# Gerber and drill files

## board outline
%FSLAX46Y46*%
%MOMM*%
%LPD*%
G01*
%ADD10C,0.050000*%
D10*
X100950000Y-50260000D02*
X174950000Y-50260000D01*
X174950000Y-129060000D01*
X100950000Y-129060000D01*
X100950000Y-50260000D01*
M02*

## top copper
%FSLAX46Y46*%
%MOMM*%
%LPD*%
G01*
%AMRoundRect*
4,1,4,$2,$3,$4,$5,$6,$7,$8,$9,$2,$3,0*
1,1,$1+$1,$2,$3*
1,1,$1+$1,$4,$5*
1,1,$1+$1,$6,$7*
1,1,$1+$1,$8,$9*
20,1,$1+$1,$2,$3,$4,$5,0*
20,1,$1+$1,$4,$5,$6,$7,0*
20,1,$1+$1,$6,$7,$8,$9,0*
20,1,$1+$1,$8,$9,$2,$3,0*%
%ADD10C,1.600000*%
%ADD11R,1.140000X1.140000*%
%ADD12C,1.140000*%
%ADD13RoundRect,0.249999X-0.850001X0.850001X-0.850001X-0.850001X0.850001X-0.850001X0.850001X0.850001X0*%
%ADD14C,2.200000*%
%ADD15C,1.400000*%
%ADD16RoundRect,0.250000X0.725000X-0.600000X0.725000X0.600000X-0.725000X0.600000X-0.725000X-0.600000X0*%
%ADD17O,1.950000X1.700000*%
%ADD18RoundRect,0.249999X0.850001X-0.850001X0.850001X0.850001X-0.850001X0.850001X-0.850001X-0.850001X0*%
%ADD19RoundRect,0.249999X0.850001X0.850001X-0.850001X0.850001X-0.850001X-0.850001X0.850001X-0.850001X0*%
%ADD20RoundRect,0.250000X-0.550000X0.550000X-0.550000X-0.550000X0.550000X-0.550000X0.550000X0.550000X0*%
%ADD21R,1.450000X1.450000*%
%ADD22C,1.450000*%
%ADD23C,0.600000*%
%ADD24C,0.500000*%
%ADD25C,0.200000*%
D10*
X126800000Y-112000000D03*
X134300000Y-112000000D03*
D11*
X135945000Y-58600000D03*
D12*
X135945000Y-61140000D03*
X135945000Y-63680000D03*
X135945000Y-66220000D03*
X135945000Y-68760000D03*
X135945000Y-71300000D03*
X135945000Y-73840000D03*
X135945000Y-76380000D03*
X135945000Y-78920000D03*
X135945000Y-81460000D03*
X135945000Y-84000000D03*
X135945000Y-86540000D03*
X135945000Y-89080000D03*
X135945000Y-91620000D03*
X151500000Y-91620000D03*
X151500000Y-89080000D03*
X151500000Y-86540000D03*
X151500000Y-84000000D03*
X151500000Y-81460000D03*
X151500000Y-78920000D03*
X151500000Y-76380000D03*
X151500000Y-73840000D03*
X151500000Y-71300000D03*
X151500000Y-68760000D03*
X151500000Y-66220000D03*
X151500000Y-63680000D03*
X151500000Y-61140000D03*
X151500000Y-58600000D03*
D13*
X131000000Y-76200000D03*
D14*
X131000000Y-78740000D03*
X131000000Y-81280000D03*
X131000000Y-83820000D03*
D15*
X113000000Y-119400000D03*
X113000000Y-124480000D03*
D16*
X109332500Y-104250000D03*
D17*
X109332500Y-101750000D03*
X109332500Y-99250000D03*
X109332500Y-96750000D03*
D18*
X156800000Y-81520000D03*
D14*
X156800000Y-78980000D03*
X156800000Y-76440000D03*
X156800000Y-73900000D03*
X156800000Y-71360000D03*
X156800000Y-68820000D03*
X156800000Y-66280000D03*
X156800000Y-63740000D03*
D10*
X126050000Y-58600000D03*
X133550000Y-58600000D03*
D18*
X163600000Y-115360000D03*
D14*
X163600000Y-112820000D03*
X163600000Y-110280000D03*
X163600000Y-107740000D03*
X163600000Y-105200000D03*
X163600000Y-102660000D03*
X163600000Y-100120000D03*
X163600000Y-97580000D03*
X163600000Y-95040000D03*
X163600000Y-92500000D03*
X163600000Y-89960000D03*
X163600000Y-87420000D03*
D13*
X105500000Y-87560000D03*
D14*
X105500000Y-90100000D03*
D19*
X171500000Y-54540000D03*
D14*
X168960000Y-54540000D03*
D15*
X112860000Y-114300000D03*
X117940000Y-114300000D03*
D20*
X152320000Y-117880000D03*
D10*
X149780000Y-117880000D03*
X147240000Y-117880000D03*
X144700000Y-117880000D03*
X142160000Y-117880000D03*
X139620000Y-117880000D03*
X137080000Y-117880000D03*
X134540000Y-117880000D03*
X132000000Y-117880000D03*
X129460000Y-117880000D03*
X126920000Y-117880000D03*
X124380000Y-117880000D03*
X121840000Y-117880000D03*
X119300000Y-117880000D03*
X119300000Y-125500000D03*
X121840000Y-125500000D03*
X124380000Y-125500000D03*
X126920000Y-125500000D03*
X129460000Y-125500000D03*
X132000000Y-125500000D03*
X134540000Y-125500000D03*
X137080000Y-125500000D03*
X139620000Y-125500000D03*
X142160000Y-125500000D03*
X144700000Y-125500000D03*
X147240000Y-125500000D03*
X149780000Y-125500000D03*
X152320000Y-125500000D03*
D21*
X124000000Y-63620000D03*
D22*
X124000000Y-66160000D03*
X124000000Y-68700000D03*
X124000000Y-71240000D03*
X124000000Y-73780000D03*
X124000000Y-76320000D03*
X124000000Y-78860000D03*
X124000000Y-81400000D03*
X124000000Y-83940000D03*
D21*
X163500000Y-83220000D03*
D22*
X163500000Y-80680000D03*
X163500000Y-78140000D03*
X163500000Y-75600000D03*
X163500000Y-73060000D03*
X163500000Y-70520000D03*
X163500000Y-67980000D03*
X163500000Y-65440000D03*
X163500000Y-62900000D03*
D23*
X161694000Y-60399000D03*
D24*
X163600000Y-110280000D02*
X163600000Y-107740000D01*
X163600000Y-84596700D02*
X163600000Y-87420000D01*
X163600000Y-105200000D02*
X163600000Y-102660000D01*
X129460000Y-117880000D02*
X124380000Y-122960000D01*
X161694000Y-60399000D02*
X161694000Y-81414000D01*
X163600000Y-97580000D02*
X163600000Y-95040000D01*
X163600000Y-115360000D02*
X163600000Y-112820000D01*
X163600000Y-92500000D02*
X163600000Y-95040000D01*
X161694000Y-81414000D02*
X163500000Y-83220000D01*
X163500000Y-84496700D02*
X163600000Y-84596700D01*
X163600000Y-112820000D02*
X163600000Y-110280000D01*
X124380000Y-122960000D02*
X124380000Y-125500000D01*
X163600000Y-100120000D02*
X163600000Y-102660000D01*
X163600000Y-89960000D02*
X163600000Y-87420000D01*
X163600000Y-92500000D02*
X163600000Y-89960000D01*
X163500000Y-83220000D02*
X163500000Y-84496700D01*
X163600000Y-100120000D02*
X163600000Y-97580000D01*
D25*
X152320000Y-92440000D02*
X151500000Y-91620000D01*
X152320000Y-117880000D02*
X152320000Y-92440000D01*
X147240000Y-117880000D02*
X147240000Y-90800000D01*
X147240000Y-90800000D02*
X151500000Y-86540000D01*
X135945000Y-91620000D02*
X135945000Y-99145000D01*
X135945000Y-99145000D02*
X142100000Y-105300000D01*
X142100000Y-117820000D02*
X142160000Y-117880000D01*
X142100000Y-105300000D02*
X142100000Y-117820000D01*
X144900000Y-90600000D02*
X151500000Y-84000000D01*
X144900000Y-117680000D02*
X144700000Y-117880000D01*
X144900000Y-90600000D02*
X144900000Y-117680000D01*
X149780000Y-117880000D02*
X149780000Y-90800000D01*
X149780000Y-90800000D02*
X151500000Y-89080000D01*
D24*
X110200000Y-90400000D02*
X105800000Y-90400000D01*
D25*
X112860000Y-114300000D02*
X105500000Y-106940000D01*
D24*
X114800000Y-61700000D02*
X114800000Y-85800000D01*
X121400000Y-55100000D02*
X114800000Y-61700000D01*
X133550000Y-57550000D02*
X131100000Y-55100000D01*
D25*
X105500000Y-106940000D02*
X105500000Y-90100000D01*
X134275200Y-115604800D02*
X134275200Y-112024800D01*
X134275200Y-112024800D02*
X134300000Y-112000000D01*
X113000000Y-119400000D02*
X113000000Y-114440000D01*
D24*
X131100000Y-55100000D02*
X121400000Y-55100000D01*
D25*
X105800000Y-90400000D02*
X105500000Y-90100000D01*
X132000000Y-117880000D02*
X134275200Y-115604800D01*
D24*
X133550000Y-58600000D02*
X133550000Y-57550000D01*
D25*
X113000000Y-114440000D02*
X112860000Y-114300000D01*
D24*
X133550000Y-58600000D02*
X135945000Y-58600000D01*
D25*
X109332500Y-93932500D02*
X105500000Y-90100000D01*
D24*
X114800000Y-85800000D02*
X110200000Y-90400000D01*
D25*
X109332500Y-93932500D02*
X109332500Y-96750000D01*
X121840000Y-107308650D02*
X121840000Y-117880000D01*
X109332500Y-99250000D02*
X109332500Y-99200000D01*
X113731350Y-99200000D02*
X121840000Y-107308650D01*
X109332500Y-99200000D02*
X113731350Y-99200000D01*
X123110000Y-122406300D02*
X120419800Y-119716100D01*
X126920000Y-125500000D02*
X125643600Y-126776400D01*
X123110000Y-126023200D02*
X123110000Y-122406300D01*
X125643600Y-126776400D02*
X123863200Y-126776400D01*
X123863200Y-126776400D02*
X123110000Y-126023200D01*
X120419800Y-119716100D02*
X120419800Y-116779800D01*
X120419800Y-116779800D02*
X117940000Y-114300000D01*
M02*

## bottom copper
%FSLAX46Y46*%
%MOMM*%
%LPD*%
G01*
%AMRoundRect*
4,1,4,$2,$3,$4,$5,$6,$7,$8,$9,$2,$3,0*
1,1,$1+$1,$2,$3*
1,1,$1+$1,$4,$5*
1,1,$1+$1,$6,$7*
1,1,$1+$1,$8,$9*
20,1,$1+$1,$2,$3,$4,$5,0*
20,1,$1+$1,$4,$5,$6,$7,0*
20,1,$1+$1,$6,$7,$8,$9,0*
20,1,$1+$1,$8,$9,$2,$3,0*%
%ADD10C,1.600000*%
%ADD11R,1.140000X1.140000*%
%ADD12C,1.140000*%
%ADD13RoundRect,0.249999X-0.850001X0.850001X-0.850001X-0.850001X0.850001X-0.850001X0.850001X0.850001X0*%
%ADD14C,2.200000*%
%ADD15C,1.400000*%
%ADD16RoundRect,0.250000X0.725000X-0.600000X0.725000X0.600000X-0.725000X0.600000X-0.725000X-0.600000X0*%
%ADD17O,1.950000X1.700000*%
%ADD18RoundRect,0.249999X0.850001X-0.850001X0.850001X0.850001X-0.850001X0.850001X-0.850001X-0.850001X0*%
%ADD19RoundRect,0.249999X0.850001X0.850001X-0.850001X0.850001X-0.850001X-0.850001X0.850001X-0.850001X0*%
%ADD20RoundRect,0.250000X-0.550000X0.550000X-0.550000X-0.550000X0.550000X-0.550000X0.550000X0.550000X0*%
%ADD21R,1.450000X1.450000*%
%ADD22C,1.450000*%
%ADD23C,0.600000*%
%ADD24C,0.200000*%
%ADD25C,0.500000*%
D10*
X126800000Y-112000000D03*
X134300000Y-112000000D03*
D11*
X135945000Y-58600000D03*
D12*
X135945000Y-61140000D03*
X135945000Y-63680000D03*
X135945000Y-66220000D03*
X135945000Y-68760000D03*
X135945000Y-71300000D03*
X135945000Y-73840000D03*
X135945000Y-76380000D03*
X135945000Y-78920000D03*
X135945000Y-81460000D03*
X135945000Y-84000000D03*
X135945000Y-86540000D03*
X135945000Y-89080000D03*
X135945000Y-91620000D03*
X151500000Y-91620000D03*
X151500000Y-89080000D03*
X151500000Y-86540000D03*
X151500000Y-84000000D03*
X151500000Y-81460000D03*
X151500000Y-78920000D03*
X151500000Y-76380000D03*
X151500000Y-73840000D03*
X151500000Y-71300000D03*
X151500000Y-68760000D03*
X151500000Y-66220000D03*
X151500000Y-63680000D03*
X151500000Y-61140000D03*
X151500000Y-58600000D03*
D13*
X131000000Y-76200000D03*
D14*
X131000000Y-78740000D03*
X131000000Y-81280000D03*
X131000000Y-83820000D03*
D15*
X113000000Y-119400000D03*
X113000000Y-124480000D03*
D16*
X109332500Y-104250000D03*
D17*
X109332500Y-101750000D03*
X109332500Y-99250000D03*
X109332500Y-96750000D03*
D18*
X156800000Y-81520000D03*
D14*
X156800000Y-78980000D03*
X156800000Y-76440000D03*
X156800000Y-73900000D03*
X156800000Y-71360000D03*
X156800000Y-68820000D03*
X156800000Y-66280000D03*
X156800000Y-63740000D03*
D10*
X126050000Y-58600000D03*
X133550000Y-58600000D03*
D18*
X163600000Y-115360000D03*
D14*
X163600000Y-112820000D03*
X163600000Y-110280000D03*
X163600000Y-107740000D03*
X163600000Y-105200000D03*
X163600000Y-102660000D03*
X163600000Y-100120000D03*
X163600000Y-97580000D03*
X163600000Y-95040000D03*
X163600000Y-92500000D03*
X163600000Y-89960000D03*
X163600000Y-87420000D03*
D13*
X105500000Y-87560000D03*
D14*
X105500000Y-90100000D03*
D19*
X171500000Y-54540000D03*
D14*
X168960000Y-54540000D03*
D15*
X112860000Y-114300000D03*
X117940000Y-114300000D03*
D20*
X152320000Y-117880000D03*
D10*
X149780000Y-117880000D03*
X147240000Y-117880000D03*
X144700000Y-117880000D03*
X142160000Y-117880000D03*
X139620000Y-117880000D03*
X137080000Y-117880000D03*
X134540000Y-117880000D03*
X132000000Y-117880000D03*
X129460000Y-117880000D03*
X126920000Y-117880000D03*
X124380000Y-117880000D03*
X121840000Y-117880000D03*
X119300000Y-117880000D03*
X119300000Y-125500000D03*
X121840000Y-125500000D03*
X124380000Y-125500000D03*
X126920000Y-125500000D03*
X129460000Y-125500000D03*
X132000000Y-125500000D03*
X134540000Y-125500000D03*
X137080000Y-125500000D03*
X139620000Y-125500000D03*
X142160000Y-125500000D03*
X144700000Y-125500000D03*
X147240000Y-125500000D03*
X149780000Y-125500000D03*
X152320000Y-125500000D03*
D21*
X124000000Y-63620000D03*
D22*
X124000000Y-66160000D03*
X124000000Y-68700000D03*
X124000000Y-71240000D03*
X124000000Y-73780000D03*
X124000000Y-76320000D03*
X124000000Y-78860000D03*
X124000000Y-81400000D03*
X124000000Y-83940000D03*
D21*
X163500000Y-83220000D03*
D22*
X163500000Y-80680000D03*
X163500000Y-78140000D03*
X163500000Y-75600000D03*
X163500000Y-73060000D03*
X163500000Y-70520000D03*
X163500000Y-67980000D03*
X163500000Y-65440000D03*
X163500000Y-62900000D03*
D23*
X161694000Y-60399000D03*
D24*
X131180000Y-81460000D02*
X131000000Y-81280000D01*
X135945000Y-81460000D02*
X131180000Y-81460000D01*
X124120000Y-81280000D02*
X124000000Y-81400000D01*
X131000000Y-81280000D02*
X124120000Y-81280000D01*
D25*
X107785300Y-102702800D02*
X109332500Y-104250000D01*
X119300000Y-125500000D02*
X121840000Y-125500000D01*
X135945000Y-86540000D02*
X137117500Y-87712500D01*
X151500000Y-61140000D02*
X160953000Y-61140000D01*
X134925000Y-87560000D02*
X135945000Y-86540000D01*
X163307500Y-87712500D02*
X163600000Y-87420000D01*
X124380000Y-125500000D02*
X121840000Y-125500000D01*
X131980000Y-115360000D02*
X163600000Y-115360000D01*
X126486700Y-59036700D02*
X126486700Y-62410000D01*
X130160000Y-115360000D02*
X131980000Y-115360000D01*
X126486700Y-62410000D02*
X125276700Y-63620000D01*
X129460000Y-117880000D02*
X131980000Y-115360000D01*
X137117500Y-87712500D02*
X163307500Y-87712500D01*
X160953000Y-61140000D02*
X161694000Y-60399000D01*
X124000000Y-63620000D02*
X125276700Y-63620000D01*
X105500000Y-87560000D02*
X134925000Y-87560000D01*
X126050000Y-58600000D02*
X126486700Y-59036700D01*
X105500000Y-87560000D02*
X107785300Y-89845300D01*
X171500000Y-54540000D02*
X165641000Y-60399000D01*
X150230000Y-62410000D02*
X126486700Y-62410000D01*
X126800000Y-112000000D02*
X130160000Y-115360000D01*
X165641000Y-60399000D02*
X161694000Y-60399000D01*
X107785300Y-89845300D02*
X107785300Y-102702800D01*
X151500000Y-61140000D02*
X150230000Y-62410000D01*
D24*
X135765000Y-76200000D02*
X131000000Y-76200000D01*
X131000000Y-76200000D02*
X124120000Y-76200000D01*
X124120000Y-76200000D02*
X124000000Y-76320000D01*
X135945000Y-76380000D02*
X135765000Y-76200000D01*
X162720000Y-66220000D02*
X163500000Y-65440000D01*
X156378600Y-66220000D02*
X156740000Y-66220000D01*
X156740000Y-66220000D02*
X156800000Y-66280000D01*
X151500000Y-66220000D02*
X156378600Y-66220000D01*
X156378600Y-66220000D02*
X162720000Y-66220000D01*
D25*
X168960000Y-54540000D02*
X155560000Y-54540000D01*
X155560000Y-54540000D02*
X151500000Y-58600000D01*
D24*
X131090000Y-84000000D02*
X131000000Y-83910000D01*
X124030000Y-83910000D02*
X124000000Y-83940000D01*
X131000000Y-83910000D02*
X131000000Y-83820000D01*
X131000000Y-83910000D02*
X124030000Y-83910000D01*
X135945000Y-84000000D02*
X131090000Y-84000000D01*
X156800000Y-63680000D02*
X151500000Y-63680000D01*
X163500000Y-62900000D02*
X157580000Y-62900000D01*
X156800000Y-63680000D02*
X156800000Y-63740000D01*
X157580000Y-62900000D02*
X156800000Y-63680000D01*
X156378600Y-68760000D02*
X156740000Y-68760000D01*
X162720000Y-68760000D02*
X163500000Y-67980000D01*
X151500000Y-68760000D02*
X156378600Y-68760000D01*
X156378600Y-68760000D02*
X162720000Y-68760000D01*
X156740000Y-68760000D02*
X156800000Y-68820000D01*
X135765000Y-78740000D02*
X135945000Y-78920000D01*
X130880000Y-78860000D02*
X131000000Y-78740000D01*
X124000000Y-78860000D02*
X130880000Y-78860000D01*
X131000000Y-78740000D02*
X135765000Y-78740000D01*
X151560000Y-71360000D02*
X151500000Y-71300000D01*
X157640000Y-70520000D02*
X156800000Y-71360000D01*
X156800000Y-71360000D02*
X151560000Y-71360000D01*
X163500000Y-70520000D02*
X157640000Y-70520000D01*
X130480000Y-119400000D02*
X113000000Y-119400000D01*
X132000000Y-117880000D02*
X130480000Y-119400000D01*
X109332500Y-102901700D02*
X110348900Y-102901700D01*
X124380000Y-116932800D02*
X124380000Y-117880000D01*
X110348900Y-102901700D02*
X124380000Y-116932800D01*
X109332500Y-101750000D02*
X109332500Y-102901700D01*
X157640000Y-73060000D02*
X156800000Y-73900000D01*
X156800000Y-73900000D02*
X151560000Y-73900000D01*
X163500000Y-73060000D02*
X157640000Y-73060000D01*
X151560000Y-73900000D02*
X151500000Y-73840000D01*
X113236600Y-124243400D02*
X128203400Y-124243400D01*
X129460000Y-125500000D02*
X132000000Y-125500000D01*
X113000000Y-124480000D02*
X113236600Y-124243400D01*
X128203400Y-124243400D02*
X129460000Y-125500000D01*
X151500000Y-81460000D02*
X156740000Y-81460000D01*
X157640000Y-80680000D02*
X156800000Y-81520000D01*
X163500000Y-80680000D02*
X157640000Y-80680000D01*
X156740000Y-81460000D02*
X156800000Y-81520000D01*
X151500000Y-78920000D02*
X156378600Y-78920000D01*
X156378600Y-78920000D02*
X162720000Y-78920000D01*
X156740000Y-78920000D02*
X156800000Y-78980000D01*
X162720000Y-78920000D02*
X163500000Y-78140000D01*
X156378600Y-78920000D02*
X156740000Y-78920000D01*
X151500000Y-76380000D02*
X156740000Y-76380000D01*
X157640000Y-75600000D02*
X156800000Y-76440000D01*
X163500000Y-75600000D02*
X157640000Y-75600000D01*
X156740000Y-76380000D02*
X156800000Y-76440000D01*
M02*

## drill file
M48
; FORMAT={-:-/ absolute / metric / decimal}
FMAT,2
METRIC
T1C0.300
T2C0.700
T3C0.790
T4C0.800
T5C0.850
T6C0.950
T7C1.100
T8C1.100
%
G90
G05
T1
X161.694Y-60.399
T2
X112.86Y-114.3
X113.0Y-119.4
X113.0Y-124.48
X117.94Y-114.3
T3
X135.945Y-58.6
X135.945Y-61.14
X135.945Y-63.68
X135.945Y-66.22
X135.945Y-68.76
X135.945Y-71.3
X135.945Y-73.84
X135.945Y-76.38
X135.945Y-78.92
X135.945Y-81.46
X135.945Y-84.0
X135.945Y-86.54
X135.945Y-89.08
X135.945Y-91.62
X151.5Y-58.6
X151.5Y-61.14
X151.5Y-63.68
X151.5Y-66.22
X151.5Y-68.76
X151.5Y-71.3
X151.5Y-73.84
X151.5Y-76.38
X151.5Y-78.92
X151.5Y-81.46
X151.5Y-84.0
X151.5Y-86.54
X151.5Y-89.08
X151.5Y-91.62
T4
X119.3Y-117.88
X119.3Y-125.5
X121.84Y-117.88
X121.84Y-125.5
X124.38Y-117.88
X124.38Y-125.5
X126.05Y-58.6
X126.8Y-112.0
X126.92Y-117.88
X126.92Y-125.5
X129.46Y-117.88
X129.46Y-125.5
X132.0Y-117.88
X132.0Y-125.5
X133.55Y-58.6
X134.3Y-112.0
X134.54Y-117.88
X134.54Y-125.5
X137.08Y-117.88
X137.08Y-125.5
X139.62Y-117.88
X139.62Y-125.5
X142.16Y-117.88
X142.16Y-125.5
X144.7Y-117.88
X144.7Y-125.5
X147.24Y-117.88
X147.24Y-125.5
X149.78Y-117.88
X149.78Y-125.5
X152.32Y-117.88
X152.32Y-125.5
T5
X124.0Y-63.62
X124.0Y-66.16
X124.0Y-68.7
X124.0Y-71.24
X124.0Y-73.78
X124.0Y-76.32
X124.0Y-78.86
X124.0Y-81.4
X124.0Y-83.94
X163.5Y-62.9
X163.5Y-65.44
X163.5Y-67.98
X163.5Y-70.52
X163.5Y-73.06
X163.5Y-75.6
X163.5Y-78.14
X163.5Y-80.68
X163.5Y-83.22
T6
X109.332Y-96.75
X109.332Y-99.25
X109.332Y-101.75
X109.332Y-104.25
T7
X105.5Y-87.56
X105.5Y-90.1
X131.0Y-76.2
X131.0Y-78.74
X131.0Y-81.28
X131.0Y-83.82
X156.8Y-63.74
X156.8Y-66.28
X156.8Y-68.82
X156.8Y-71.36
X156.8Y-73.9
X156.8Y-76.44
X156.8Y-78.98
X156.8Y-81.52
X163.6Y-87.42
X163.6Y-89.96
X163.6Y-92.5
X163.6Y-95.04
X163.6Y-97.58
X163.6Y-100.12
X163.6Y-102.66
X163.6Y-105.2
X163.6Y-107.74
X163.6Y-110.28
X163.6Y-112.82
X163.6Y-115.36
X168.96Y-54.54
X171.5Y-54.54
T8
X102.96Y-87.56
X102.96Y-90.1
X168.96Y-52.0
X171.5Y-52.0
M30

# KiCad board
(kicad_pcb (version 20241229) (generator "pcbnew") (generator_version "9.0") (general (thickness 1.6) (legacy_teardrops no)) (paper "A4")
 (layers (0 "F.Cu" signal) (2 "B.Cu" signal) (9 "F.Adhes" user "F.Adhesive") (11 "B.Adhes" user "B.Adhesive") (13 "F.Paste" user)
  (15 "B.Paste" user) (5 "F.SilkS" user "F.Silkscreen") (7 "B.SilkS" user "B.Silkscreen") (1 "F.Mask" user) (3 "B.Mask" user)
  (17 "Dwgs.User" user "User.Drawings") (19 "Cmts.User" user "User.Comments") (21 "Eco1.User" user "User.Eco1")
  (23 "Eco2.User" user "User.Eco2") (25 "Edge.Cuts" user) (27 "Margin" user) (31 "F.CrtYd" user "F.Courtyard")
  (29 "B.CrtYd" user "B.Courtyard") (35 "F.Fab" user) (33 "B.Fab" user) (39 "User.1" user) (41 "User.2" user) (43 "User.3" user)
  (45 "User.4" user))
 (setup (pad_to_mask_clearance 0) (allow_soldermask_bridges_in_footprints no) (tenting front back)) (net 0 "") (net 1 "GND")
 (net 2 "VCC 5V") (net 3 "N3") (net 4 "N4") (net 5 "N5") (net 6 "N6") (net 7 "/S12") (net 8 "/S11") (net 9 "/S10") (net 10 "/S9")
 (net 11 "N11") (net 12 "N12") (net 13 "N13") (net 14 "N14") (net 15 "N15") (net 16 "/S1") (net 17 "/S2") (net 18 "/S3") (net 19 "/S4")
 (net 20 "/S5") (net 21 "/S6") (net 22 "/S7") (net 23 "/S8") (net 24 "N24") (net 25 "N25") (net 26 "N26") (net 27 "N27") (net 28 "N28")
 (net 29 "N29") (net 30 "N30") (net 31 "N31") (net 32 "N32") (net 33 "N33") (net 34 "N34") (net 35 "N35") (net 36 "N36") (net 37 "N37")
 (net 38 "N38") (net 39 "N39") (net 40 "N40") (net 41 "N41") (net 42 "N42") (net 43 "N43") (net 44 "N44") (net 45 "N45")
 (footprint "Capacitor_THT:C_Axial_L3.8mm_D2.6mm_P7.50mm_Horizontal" (layer "F.Cu") (at 126.8 112)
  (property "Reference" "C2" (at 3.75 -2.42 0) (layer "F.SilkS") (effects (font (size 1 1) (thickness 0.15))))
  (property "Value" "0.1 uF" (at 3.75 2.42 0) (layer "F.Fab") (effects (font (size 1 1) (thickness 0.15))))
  (pad "1" thru_hole circle (at 0 0) (size 1.6 1.6) (drill 0.8) (layers "*.Cu" "*.Mask") (remove_unused_layers no) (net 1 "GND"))
  (pad "2" thru_hole circle (at 7.5 0) (size 1.6 1.6) (drill 0.8) (layers "*.Cu" "*.Mask") (remove_unused_layers no) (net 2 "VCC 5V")))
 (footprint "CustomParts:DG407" (layer "F.Cu") (at 143.7225 75.11)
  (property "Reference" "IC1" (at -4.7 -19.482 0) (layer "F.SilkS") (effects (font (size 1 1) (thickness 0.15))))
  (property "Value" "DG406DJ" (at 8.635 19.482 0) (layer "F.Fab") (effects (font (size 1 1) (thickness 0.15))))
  (pad "1" thru_hole rect (at -7.7775 -16.51) (size 1.14 1.14) (drill 0.79) (layers "*.Cu" "*.Mask") (remove_unused_layers no)
   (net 2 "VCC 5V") (solder_mask_margin 0.102))
  (pad "2" thru_hole circle (at -7.7775 -13.97) (size 1.14 1.14) (drill 0.79) (layers "*.Cu" "*.Mask") (remove_unused_layers no)
   (solder_mask_margin 0.102))
  (pad "3" thru_hole circle (at -7.7775 -11.43) (size 1.14 1.14) (drill 0.79) (layers "*.Cu" "*.Mask") (remove_unused_layers no)
   (solder_mask_margin 0.102))
  (pad "4" thru_hole circle (at -7.7775 -8.89) (size 1.14 1.14) (drill 0.79) (layers "*.Cu" "*.Mask") (remove_unused_layers no) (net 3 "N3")
   (solder_mask_margin 0.102))
  (pad "5" thru_hole circle (at -7.7775 -6.35) (size 1.14 1.14) (drill 0.79) (layers "*.Cu" "*.Mask") (remove_unused_layers no) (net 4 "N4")
   (solder_mask_margin 0.102))
  (pad "6" thru_hole circle (at -7.7775 -3.81) (size 1.14 1.14) (drill 0.79) (layers "*.Cu" "*.Mask") (remove_unused_layers no) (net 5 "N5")
   (solder_mask_margin 0.102))
  (pad "7" thru_hole circle (at -7.7775 -1.27) (size 1.14 1.14) (drill 0.79) (layers "*.Cu" "*.Mask") (remove_unused_layers no) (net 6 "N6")
   (solder_mask_margin 0.102))
  (pad "8" thru_hole circle (at -7.7775 1.27) (size 1.14 1.14) (drill 0.79) (layers "*.Cu" "*.Mask") (remove_unused_layers no)
   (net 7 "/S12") (solder_mask_margin 0.102))
  (pad "9" thru_hole circle (at -7.7775 3.81) (size 1.14 1.14) (drill 0.79) (layers "*.Cu" "*.Mask") (remove_unused_layers no)
   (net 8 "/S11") (solder_mask_margin 0.102))
  (pad "10" thru_hole circle (at -7.7775 6.35) (size 1.14 1.14) (drill 0.79) (layers "*.Cu" "*.Mask") (remove_unused_layers no)
   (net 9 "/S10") (solder_mask_margin 0.102))
  (pad "11" thru_hole circle (at -7.7775 8.89) (size 1.14 1.14) (drill 0.79) (layers "*.Cu" "*.Mask") (remove_unused_layers no)
   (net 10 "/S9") (solder_mask_margin 0.102))
  (pad "12" thru_hole circle (at -7.7775 11.43) (size 1.14 1.14) (drill 0.79) (layers "*.Cu" "*.Mask") (remove_unused_layers no)
   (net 1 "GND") (solder_mask_margin 0.102))
  (pad "13" thru_hole circle (at -7.7775 13.97) (size 1.14 1.14) (drill 0.79) (layers "*.Cu" "*.Mask") (remove_unused_layers no)
   (solder_mask_margin 0.102))
  (pad "14" thru_hole circle (at -7.7775 16.51) (size 1.14 1.14) (drill 0.79) (layers "*.Cu" "*.Mask") (remove_unused_layers no)
   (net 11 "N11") (solder_mask_margin 0.102))
  (pad "15" thru_hole circle (at 7.7775 16.51) (size 1.14 1.14) (drill 0.79) (layers "*.Cu" "*.Mask") (remove_unused_layers no)
   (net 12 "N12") (solder_mask_margin 0.102))
  (pad "16" thru_hole circle (at 7.7775 13.97) (size 1.14 1.14) (drill 0.79) (layers "*.Cu" "*.Mask") (remove_unused_layers no)
   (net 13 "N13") (solder_mask_margin 0.102))
  (pad "17" thru_hole circle (at 7.7775 11.43) (size 1.14 1.14) (drill 0.79) (layers "*.Cu" "*.Mask") (remove_unused_layers no)
   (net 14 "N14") (solder_mask_margin 0.102))
  (pad "18" thru_hole circle (at 7.7775 8.89) (size 1.14 1.14) (drill 0.79) (layers "*.Cu" "*.Mask") (remove_unused_layers no)
   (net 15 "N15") (solder_mask_margin 0.102))
  (pad "19" thru_hole circle (at 7.7775 6.35) (size 1.14 1.14) (drill 0.79) (layers "*.Cu" "*.Mask") (remove_unused_layers no)
   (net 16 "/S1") (solder_mask_margin 0.102))
  (pad "20" thru_hole circle (at 7.7775 3.81) (size 1.14 1.14) (drill 0.79) (layers "*.Cu" "*.Mask") (remove_unused_layers no)
   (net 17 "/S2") (solder_mask_margin 0.102))
  (pad "21" thru_hole circle (at 7.7775 1.27) (size 1.14 1.14) (drill 0.79) (layers "*.Cu" "*.Mask") (remove_unused_layers no)
   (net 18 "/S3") (solder_mask_margin 0.102))
  (pad "22" thru_hole circle (at 7.7775 -1.27) (size 1.14 1.14) (drill 0.79) (layers "*.Cu" "*.Mask") (remove_unused_layers no)
   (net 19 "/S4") (solder_mask_margin 0.102))
  (pad "23" thru_hole circle (at 7.7775 -3.81) (size 1.14 1.14) (drill 0.79) (layers "*.Cu" "*.Mask") (remove_unused_layers no)
   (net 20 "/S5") (solder_mask_margin 0.102))
  (pad "24" thru_hole circle (at 7.7775 -6.35) (size 1.14 1.14) (drill 0.79) (layers "*.Cu" "*.Mask") (remove_unused_layers no)
   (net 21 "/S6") (solder_mask_margin 0.102))
  (pad "25" thru_hole circle (at 7.7775 -8.89) (size 1.14 1.14) (drill 0.79) (layers "*.Cu" "*.Mask") (remove_unused_layers no)
   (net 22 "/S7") (solder_mask_margin 0.102))
  (pad "26" thru_hole circle (at 7.7775 -11.43) (size 1.14 1.14) (drill 0.79) (layers "*.Cu" "*.Mask") (remove_unused_layers no)
   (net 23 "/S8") (solder_mask_margin 0.102))
  (pad "27" thru_hole circle (at 7.7775 -13.97) (size 1.14 1.14) (drill 0.79) (layers "*.Cu" "*.Mask") (remove_unused_layers no)
   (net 1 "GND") (solder_mask_margin 0.102))
  (pad "28" thru_hole circle (at 7.7775 -16.51) (size 1.14 1.14) (drill 0.79) (layers "*.Cu" "*.Mask") (remove_unused_layers no)
   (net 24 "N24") (solder_mask_margin 0.102)))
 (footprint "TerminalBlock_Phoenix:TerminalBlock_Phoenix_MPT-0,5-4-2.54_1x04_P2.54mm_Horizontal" (layer "F.Cu") (at 131 76.2 -90)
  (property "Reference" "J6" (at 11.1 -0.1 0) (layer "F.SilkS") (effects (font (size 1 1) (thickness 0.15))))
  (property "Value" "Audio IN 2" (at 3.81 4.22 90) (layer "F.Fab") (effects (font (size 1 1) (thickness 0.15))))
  (pad "1" thru_hole roundrect (at 0 0 270) (size 2.2 2.2) (drill 1.1) (layers "*.Cu" "*.Mask") (remove_unused_layers no)
   (roundrect_rratio 0.113636) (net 7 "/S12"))
  (pad "2" thru_hole circle (at 2.54 0 270) (size 2.2 2.2) (drill 1.1) (layers "*.Cu" "*.Mask") (remove_unused_layers no) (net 8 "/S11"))
  (pad "3" thru_hole circle (at 5.08 0 270) (size 2.2 2.2) (drill 1.1) (layers "*.Cu" "*.Mask") (remove_unused_layers no) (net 9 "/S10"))
  (pad "4" thru_hole circle (at 7.62 0 270) (size 2.2 2.2) (drill 1.1) (layers "*.Cu" "*.Mask") (remove_unused_layers no) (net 10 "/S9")))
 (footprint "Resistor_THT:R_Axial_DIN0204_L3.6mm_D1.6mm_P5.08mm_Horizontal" (layer "F.Cu") (at 113 119.4 -90)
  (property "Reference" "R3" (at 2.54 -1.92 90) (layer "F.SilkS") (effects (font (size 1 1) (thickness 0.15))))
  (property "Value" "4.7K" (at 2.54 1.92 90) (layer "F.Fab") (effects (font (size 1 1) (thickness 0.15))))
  (pad "1" thru_hole circle (at 0 0 270) (size 1.4 1.4) (drill 0.7) (layers "*.Cu" "*.Mask") (remove_unused_layers no) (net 2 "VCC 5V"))
  (pad "2" thru_hole circle (at 5.08 0 270) (size 1.4 1.4) (drill 0.7) (layers "*.Cu" "*.Mask") (remove_unused_layers no) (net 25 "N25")))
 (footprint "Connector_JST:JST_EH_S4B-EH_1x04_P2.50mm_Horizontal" (layer "F.Cu") (at 109.3325 104.25 90)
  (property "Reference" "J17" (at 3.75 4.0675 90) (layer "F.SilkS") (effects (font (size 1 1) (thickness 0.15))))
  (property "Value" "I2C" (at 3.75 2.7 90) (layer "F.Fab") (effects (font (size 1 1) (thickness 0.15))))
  (pad "1" thru_hole roundrect (at 0 0 90) (size 1.7 1.95) (drill 0.95) (layers "*.Cu" "*.Mask") (remove_unused_layers no)
   (roundrect_rratio 0.147059) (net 1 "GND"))
  (pad "2" thru_hole oval (at 2.5 0 90) (size 1.7 1.95) (drill 0.95) (layers "*.Cu" "*.Mask") (remove_unused_layers no) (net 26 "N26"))
  (pad "3" thru_hole oval (at 5 0 90) (size 1.7 1.95) (drill 0.95) (layers "*.Cu" "*.Mask") (remove_unused_layers no) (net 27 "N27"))
  (pad "4" thru_hole oval (at 7.5 0 90) (size 1.7 1.95) (drill 0.95) (layers "*.Cu" "*.Mask") (remove_unused_layers no) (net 2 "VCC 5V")))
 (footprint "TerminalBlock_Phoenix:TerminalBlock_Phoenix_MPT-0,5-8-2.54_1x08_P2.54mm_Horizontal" (layer "F.Cu") (at 156.8 81.52 90)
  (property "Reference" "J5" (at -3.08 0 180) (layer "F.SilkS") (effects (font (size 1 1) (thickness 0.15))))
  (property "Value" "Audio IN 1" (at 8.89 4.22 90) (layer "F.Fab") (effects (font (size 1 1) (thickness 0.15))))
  (pad "1" thru_hole roundrect (at 0 0 90) (size 2.2 2.2) (drill 1.1) (layers "*.Cu" "*.Mask") (remove_unused_layers no)
   (roundrect_rratio 0.113636) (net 16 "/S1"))
  (pad "2" thru_hole circle (at 2.54 0 90) (size 2.2 2.2) (drill 1.1) (layers "*.Cu" "*.Mask") (remove_unused_layers no) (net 17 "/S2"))
  (pad "3" thru_hole circle (at 5.08 0 90) (size 2.2 2.2) (drill 1.1) (layers "*.Cu" "*.Mask") (remove_unused_layers no) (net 18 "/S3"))
  (pad "4" thru_hole circle (at 7.62 0 90) (size 2.2 2.2) (drill 1.1) (layers "*.Cu" "*.Mask") (remove_unused_layers no) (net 19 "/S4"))
  (pad "5" thru_hole circle (at 10.16 0 90) (size 2.2 2.2) (drill 1.1) (layers "*.Cu" "*.Mask") (remove_unused_layers no) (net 20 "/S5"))
  (pad "6" thru_hole circle (at 12.7 0 90) (size 2.2 2.2) (drill 1.1) (layers "*.Cu" "*.Mask") (remove_unused_layers no) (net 21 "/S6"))
  (pad "7" thru_hole circle (at 15.24 0 90) (size 2.2 2.2) (drill 1.1) (layers "*.Cu" "*.Mask") (remove_unused_layers no) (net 22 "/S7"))
  (pad "8" thru_hole circle (at 17.78 0 90) (size 2.2 2.2) (drill 1.1) (layers "*.Cu" "*.Mask") (remove_unused_layers no) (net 23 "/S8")))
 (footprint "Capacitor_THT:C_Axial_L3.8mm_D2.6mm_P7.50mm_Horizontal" (layer "F.Cu") (at 126.05 58.6)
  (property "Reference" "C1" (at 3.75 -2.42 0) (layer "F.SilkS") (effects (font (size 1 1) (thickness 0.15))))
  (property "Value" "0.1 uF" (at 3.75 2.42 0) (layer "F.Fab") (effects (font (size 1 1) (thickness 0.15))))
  (pad "1" thru_hole circle (at 0 0) (size 1.6 1.6) (drill 0.8) (layers "*.Cu" "*.Mask") (remove_unused_layers no) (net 1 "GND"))
  (pad "2" thru_hole circle (at 7.5 0) (size 1.6 1.6) (drill 0.8) (layers "*.Cu" "*.Mask") (remove_unused_layers no) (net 2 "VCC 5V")))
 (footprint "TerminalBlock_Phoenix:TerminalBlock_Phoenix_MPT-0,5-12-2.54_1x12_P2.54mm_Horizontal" (layer "F.Cu") (at 163.6 115.36 90)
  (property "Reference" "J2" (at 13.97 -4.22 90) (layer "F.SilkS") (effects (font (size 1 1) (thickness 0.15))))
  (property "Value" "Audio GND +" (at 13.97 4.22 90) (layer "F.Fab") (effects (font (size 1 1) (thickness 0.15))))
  (pad "1" thru_hole roundrect (at 0 0 90) (size 2.2 2.2) (drill 1.1) (layers "*.Cu" "*.Mask") (remove_unused_layers no)
   (roundrect_rratio 0.113636) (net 1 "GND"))
  (pad "2" thru_hole circle (at 2.54 0 90) (size 2.2 2.2) (drill 1.1) (layers "*.Cu" "*.Mask") (remove_unused_layers no) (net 1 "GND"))
  (pad "3" thru_hole circle (at 5.08 0 90) (size 2.2 2.2) (drill 1.1) (layers "*.Cu" "*.Mask") (remove_unused_layers no) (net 1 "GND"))
  (pad "4" thru_hole circle (at 7.62 0 90) (size 2.2 2.2) (drill 1.1) (layers "*.Cu" "*.Mask") (remove_unused_layers no) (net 1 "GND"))
  (pad "5" thru_hole circle (at 10.16 0 90) (size 2.2 2.2) (drill 1.1) (layers "*.Cu" "*.Mask") (remove_unused_layers no) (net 1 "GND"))
  (pad "6" thru_hole circle (at 12.7 0 90) (size 2.2 2.2) (drill 1.1) (layers "*.Cu" "*.Mask") (remove_unused_layers no) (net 1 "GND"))
  (pad "7" thru_hole circle (at 15.24 0 90) (size 2.2 2.2) (drill 1.1) (layers "*.Cu" "*.Mask") (remove_unused_layers no) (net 1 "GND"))
  (pad "8" thru_hole circle (at 17.78 0 90) (size 2.2 2.2) (drill 1.1) (layers "*.Cu" "*.Mask") (remove_unused_layers no) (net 1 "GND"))
  (pad "9" thru_hole circle (at 20.32 0 90) (size 2.2 2.2) (drill 1.1) (layers "*.Cu" "*.Mask") (remove_unused_layers no) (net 1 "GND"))
  (pad "10" thru_hole circle (at 22.86 0 90) (size 2.2 2.2) (drill 1.1) (layers "*.Cu" "*.Mask") (remove_unused_layers no) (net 1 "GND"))
  (pad "11" thru_hole circle (at 25.4 0 90) (size 2.2 2.2) (drill 1.1) (layers "*.Cu" "*.Mask") (remove_unused_layers no) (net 1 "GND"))
  (pad "12" thru_hole circle (at 27.94 0 90) (size 2.2 2.2) (drill 1.1) (layers "*.Cu" "*.Mask") (remove_unused_layers no) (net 1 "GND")))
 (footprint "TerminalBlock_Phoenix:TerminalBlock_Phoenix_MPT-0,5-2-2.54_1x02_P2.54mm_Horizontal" (layer "F.Cu") (at 105.5 87.56 -90)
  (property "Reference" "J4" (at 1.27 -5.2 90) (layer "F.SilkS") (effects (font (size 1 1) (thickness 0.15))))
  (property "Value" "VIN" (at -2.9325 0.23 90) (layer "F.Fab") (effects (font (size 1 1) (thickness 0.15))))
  (pad "" np_thru_hole circle (at 0 2.54 270) (size 1.1 1.1) (drill 1.1) (layers "*.Cu" "*.Mask"))
  (pad "" np_thru_hole circle (at 2.54 2.54 270) (size 1.1 1.1) (drill 1.1) (layers "*.Cu" "*.Mask"))
  (pad "1" thru_hole roundrect (at 0 0 270) (size 2.2 2.2) (drill 1.1) (layers "*.Cu" "*.Mask") (remove_unused_layers no)
   (roundrect_rratio 0.113636) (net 1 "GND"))
  (pad "2" thru_hole circle (at 2.54 0 270) (size 2.2 2.2) (drill 1.1) (layers "*.Cu" "*.Mask") (remove_unused_layers no) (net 2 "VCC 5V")))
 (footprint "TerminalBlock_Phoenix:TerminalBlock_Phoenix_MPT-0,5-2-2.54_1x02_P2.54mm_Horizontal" (layer "F.Cu") (at 171.5 54.54 180)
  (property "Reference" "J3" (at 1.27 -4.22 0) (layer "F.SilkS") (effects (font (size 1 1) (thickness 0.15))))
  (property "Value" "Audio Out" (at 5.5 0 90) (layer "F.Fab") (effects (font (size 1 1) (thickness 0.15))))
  (pad "" np_thru_hole circle (at 0 2.54 180) (size 1.1 1.1) (drill 1.1) (layers "*.Cu" "*.Mask"))
  (pad "" np_thru_hole circle (at 2.54 2.54 180) (size 1.1 1.1) (drill 1.1) (layers "*.Cu" "*.Mask"))
  (pad "1" thru_hole roundrect (at 0 0 180) (size 2.2 2.2) (drill 1.1) (layers "*.Cu" "*.Mask") (remove_unused_layers no)
   (roundrect_rratio 0.113636) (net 1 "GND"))
  (pad "2" thru_hole circle (at 2.54 0 180) (size 2.2 2.2) (drill 1.1) (layers "*.Cu" "*.Mask") (remove_unused_layers no) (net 24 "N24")))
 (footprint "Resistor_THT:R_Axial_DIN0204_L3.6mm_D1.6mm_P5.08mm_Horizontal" (layer "F.Cu") (at 112.86 114.3)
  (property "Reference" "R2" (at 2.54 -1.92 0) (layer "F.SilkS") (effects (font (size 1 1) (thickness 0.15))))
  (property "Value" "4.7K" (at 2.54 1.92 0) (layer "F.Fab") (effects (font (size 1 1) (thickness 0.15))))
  (pad "1" thru_hole circle (at 0 0) (size 1.4 1.4) (drill 0.7) (layers "*.Cu" "*.Mask") (remove_unused_layers no) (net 2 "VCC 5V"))
  (pad "2" thru_hole circle (at 5.08 0) (size 1.4 1.4) (drill 0.7) (layers "*.Cu" "*.Mask") (remove_unused_layers no) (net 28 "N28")))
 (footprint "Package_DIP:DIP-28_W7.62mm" (layer "F.Cu") (at 152.32 117.88 -90)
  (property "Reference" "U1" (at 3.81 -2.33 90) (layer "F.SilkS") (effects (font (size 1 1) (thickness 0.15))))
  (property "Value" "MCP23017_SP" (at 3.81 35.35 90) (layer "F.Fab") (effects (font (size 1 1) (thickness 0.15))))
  (pad "1" thru_hole roundrect (at 0 0 270) (size 1.6 1.6) (drill 0.8) (layers "*.Cu" "*.Mask") (remove_unused_layers no)
   (roundrect_rratio 0.15625) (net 12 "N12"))
  (pad "2" thru_hole circle (at 0 2.54 270) (size 1.6 1.6) (drill 0.8) (layers "*.Cu" "*.Mask") (remove_unused_layers no) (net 13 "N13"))
  (pad "3" thru_hole circle (at 0 5.08 270) (size 1.6 1.6) (drill 0.8) (layers "*.Cu" "*.Mask") (remove_unused_layers no) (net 14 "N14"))
  (pad "4" thru_hole circle (at 0 7.62 270) (size 1.6 1.6) (drill 0.8) (layers "*.Cu" "*.Mask") (remove_unused_layers no) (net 15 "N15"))
  (pad "5" thru_hole circle (at 0 10.16 270) (size 1.6 1.6) (drill 0.8) (layers "*.Cu" "*.Mask") (remove_unused_layers no) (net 11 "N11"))
  (pad "6" thru_hole circle (at 0 12.7 270) (size 1.6 1.6) (drill 0.8) (layers "*.Cu" "*.Mask") (remove_unused_layers no) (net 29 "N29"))
  (pad "7" thru_hole circle (at 0 15.24 270) (size 1.6 1.6) (drill 0.8) (layers "*.Cu" "*.Mask") (remove_unused_layers no) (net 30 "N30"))
  (pad "8" thru_hole circle (at 0 17.78 270) (size 1.6 1.6) (drill 0.8) (layers "*.Cu" "*.Mask") (remove_unused_layers no) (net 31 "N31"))
  (pad "9" thru_hole circle (at 0 20.32 270) (size 1.6 1.6) (drill 0.8) (layers "*.Cu" "*.Mask") (remove_unused_layers no) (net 2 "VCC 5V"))
  (pad "10" thru_hole circle (at 0 22.86 270) (size 1.6 1.6) (drill 0.8) (layers "*.Cu" "*.Mask") (remove_unused_layers no) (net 1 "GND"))
  (pad "11" thru_hole circle (at 0 25.4 270) (size 1.6 1.6) (drill 0.8) (layers "*.Cu" "*.Mask") (remove_unused_layers no) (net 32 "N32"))
  (pad "12" thru_hole circle (at 0 27.94 270) (size 1.6 1.6) (drill 0.8) (layers "*.Cu" "*.Mask") (remove_unused_layers no) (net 26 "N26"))
  (pad "13" thru_hole circle (at 0 30.48 270) (size 1.6 1.6) (drill 0.8) (layers "*.Cu" "*.Mask") (remove_unused_layers no) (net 27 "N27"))
  (pad "14" thru_hole circle (at 0 33.02 270) (size 1.6 1.6) (drill 0.8) (layers "*.Cu" "*.Mask") (remove_unused_layers no) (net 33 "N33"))
  (pad "15" thru_hole circle (at 7.62 33.02 270) (size 1.6 1.6) (drill 0.8) (layers "*.Cu" "*.Mask") (remove_unused_layers no) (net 1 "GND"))
  (pad "16" thru_hole circle (at 7.62 30.48 270) (size 1.6 1.6) (drill 0.8) (layers "*.Cu" "*.Mask") (remove_unused_layers no) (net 1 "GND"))
  (pad "17" thru_hole circle (at 7.62 27.94 270) (size 1.6 1.6) (drill 0.8) (layers "*.Cu" "*.Mask") (remove_unused_layers no) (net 1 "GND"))
  (pad "18" thru_hole circle (at 7.62 25.4 270) (size 1.6 1.6) (drill 0.8) (layers "*.Cu" "*.Mask") (remove_unused_layers no) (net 28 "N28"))
  (pad "19" thru_hole circle (at 7.62 22.86 270) (size 1.6 1.6) (drill 0.8) (layers "*.Cu" "*.Mask") (remove_unused_layers no)
   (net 25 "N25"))
  (pad "20" thru_hole circle (at 7.62 20.32 270) (size 1.6 1.6) (drill 0.8) (layers "*.Cu" "*.Mask") (remove_unused_layers no)
   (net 25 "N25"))
  (pad "21" thru_hole circle (at 7.62 17.78 270) (size 1.6 1.6) (drill 0.8) (layers "*.Cu" "*.Mask") (remove_unused_layers no)
   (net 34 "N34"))
  (pad "22" thru_hole circle (at 7.62 15.24 270) (size 1.6 1.6) (drill 0.8) (layers "*.Cu" "*.Mask") (remove_unused_layers no)
   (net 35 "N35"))
  (pad "23" thru_hole circle (at 7.62 12.7 270) (size 1.6 1.6) (drill 0.8) (layers "*.Cu" "*.Mask") (remove_unused_layers no) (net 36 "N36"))
  (pad "24" thru_hole circle (at 7.62 10.16 270) (size 1.6 1.6) (drill 0.8) (layers "*.Cu" "*.Mask") (remove_unused_layers no)
   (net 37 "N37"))
  (pad "25" thru_hole circle (at 7.62 7.62 270) (size 1.6 1.6) (drill 0.8) (layers "*.Cu" "*.Mask") (remove_unused_layers no) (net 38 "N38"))
  (pad "26" thru_hole circle (at 7.62 5.08 270) (size 1.6 1.6) (drill 0.8) (layers "*.Cu" "*.Mask") (remove_unused_layers no) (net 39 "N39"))
  (pad "27" thru_hole circle (at 7.62 2.54 270) (size 1.6 1.6) (drill 0.8) (layers "*.Cu" "*.Mask") (remove_unused_layers no) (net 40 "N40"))
  (pad "28" thru_hole circle (at 7.62 0 270) (size 1.6 1.6) (drill 0.8) (layers "*.Cu" "*.Mask") (remove_unused_layers no) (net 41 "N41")))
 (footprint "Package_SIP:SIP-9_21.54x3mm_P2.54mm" (layer "B.Cu") (at 124 63.62 -90)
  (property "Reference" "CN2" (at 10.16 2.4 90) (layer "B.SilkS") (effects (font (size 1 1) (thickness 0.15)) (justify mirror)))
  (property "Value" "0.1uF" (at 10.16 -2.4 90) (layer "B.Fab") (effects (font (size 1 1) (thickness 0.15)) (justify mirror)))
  (pad "1" thru_hole rect (at 0 0 180) (size 1.45 1.45) (drill 0.85) (layers "*.Cu" "*.Mask") (remove_unused_layers no) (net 1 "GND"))
  (pad "2" thru_hole circle (at 2.54 0 180) (size 1.45 1.45) (drill 0.85) (layers "*.Cu" "*.Mask") (remove_unused_layers no) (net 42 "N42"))
  (pad "3" thru_hole circle (at 5.08 0 180) (size 1.45 1.45) (drill 0.85) (layers "*.Cu" "*.Mask") (remove_unused_layers no) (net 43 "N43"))
  (pad "4" thru_hole circle (at 7.62 0 180) (size 1.45 1.45) (drill 0.85) (layers "*.Cu" "*.Mask") (remove_unused_layers no) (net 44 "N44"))
  (pad "5" thru_hole circle (at 10.16 0 180) (size 1.45 1.45) (drill 0.85) (layers "*.Cu" "*.Mask") (remove_unused_layers no) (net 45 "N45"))
  (pad "6" thru_hole circle (at 12.7 0 180) (size 1.45 1.45) (drill 0.85) (layers "*.Cu" "*.Mask") (remove_unused_layers no) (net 7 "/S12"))
  (pad "7" thru_hole circle (at 15.24 0 180) (size 1.45 1.45) (drill 0.85) (layers "*.Cu" "*.Mask") (remove_unused_layers no) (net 8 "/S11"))
  (pad "8" thru_hole circle (at 17.78 0 180) (size 1.45 1.45) (drill 0.85) (layers "*.Cu" "*.Mask") (remove_unused_layers no) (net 9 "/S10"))
  (pad "9" thru_hole circle (at 20.32 0 180) (size 1.45 1.45) (drill 0.85) (layers "*.Cu" "*.Mask") (remove_unused_layers no) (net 10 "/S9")))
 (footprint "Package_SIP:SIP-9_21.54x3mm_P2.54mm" (layer "B.Cu") (at 163.5 83.22 90)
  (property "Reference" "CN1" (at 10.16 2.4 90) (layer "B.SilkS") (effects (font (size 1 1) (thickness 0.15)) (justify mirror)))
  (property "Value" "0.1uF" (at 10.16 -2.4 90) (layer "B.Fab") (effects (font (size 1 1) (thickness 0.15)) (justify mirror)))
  (pad "1" thru_hole rect (at 0 0) (size 1.45 1.45) (drill 0.85) (layers "*.Cu" "*.Mask") (remove_unused_layers no) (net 1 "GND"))
  (pad "2" thru_hole circle (at 2.54 0) (size 1.45 1.45) (drill 0.85) (layers "*.Cu" "*.Mask") (remove_unused_layers no) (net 16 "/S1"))
  (pad "3" thru_hole circle (at 5.08 0) (size 1.45 1.45) (drill 0.85) (layers "*.Cu" "*.Mask") (remove_unused_layers no) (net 17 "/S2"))
  (pad "4" thru_hole circle (at 7.62 0) (size 1.45 1.45) (drill 0.85) (layers "*.Cu" "*.Mask") (remove_unused_layers no) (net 18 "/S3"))
  (pad "5" thru_hole circle (at 10.16 0) (size 1.45 1.45) (drill 0.85) (layers "*.Cu" "*.Mask") (remove_unused_layers no) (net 19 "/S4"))
  (pad "6" thru_hole circle (at 12.7 0) (size 1.45 1.45) (drill 0.85) (layers "*.Cu" "*.Mask") (remove_unused_layers no) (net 20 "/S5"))
  (pad "7" thru_hole circle (at 15.24 0) (size 1.45 1.45) (drill 0.85) (layers "*.Cu" "*.Mask") (remove_unused_layers no) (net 21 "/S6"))
  (pad "8" thru_hole circle (at 17.78 0) (size 1.45 1.45) (drill 0.85) (layers "*.Cu" "*.Mask") (remove_unused_layers no) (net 22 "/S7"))
  (pad "9" thru_hole circle (at 20.32 0) (size 1.45 1.45) (drill 0.85) (layers "*.Cu" "*.Mask") (remove_unused_layers no) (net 23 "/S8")))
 (gr_rect (start 100.95 50.26) (end 174.95 129.06) (stroke (width 0.05) (type default)) (fill no) (layer "Edge.Cuts"))
 (segment (start 131.18 81.46) (end 131 81.28) (width 0.2) (layer "B.Cu") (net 9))
 (segment (start 135.945 81.46) (end 131.18 81.46) (width 0.2) (layer "B.Cu") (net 9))
 (segment (start 124.12 81.28) (end 124 81.4) (width 0.2) (layer "B.Cu") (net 9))
 (segment (start 131 81.28) (end 124.12 81.28) (width 0.2) (layer "B.Cu") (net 9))
 (segment (start 163.6 110.28) (end 163.6 107.74) (width 0.5) (layer "F.Cu") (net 1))
 (segment (start 163.6 84.5967) (end 163.6 87.42) (width 0.5) (layer "F.Cu") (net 1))
 (segment (start 163.6 105.2) (end 163.6 102.66) (width 0.5) (layer "F.Cu") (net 1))
 (segment (start 129.46 117.88) (end 124.38 122.96) (width 0.5) (layer "F.Cu") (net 1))
 (segment (start 161.694 60.399) (end 161.694 81.414) (width 0.5) (layer "F.Cu") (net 1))
 (segment (start 163.6 97.58) (end 163.6 95.04) (width 0.5) (layer "F.Cu") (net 1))
 (segment (start 163.6 115.36) (end 163.6 112.82) (width 0.5) (layer "F.Cu") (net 1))
 (segment (start 163.6 92.5) (end 163.6 95.04) (width 0.5) (layer "F.Cu") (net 1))
 (segment (start 161.694 81.414) (end 163.5 83.22) (width 0.5) (layer "F.Cu") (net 1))
 (segment (start 163.5 84.4967) (end 163.6 84.5967) (width 0.5) (layer "F.Cu") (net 1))
 (segment (start 163.6 112.82) (end 163.6 110.28) (width 0.5) (layer "F.Cu") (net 1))
 (segment (start 124.38 122.96) (end 124.38 125.5) (width 0.5) (layer "F.Cu") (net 1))
 (segment (start 163.6 100.12) (end 163.6 102.66) (width 0.5) (layer "F.Cu") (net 1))
 (segment (start 163.6 89.96) (end 163.6 87.42) (width 0.5) (layer "F.Cu") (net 1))
 (segment (start 163.6 92.5) (end 163.6 89.96) (width 0.5) (layer "F.Cu") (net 1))
 (segment (start 163.5 83.22) (end 163.5 84.4967) (width 0.5) (layer "F.Cu") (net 1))
 (segment (start 163.6 100.12) (end 163.6 97.58) (width 0.5) (layer "F.Cu") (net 1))
 (via (at 161.694 60.399) (size 0.6) (drill 0.3) (layers "F.Cu" "B.Cu") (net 1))
 (segment (start 107.7853 102.7028) (end 109.3325 104.25) (width 0.5) (layer "B.Cu") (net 1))
 (segment (start 119.3 125.5) (end 121.84 125.5) (width 0.5) (layer "B.Cu") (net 1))
 (segment (start 135.945 86.54) (end 137.1175 87.7125) (width 0.5) (layer "B.Cu") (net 1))
 (segment (start 151.5 61.14) (end 160.953 61.14) (width 0.5) (layer "B.Cu") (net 1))
 (segment (start 134.925 87.56) (end 135.945 86.54) (width 0.5) (layer "B.Cu") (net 1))
 (segment (start 163.3075 87.7125) (end 163.6 87.42) (width 0.5) (layer "B.Cu") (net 1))
 (segment (start 124.38 125.5) (end 121.84 125.5) (width 0.5) (layer "B.Cu") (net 1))
 (segment (start 131.98 115.36) (end 163.6 115.36) (width 0.5) (layer "B.Cu") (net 1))
 (segment (start 126.4867 59.0367) (end 126.4867 62.41) (width 0.5) (layer "B.Cu") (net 1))
 (segment (start 130.16 115.36) (end 131.98 115.36) (width 0.5) (layer "B.Cu") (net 1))
 (segment (start 126.4867 62.41) (end 125.2767 63.62) (width 0.5) (layer "B.Cu") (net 1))
 (segment (start 129.46 117.88) (end 131.98 115.36) (width 0.5) (layer "B.Cu") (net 1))
 (segment (start 137.1175 87.7125) (end 163.3075 87.7125) (width 0.5) (layer "B.Cu") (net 1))
 (segment (start 160.953 61.14) (end 161.694 60.399) (width 0.5) (layer "B.Cu") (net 1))
 (segment (start 124 63.62) (end 125.2767 63.62) (width 0.5) (layer "B.Cu") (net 1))
 (segment (start 105.5 87.56) (end 134.925 87.56) (width 0.5) (layer "B.Cu") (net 1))
 (segment (start 126.05 58.6) (end 126.4867 59.0367) (width 0.5) (layer "B.Cu") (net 1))
 (segment (start 105.5 87.56) (end 107.7853 89.8453) (width 0.5) (layer "B.Cu") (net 1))
 (segment (start 171.5 54.54) (end 165.641 60.399) (width 0.5) (layer "B.Cu") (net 1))
 (segment (start 150.23 62.41) (end 126.4867 62.41) (width 0.5) (layer "B.Cu") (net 1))
 (segment (start 126.8 112) (end 130.16 115.36) (width 0.5) (layer "B.Cu") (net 1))
 (segment (start 165.641 60.399) (end 161.694 60.399) (width 0.5) (layer "B.Cu") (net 1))
 (segment (start 107.7853 89.8453) (end 107.7853 102.7028) (width 0.5) (layer "B.Cu") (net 1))
 (segment (start 151.5 61.14) (end 150.23 62.41) (width 0.5) (layer "B.Cu") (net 1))
 (segment (start 135.765 76.2) (end 131 76.2) (width 0.2) (layer "B.Cu") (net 7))
 (segment (start 131 76.2) (end 124.12 76.2) (width 0.2) (layer "B.Cu") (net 7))
 (segment (start 124.12 76.2) (end 124 76.32) (width 0.2) (layer "B.Cu") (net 7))
 (segment (start 135.945 76.38) (end 135.765 76.2) (width 0.2) (layer "B.Cu") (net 7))
 (segment (start 152.32 92.44) (end 151.5 91.62) (width 0.2) (layer "F.Cu") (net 12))
 (segment (start 152.32 117.88) (end 152.32 92.44) (width 0.2) (layer "F.Cu") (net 12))
 (segment (start 162.72 66.22) (end 163.5 65.44) (width 0.2) (layer "B.Cu") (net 22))
 (segment (start 156.3786 66.22) (end 156.74 66.22) (width 0.2) (layer "B.Cu") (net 22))
 (segment (start 156.74 66.22) (end 156.8 66.28) (width 0.2) (layer "B.Cu") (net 22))
 (segment (start 151.5 66.22) (end 156.3786 66.22) (width 0.2) (layer "B.Cu") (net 22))
 (segment (start 156.3786 66.22) (end 162.72 66.22) (width 0.2) (layer "B.Cu") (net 22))
 (segment (start 168.96 54.54) (end 155.56 54.54) (width 0.5) (layer "B.Cu") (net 24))
 (segment (start 155.56 54.54) (end 151.5 58.6) (width 0.5) (layer "B.Cu") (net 24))
 (segment (start 147.24 117.88) (end 147.24 90.8) (width 0.2) (layer "F.Cu") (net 14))
 (segment (start 147.24 90.8) (end 151.5 86.54) (width 0.2) (layer "F.Cu") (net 14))
 (segment (start 135.945 91.62) (end 135.945 99.145) (width 0.2) (layer "F.Cu") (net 11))
 (segment (start 135.945 99.145) (end 142.1 105.3) (width 0.2) (layer "F.Cu") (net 11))
 (segment (start 142.1 117.82) (end 142.16 117.88) (width 0.2) (layer "F.Cu") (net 11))
 (segment (start 142.1 105.3) (end 142.1 117.82) (width 0.2) (layer "F.Cu") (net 11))
 (segment (start 131.09 84) (end 131 83.91) (width 0.2) (layer "B.Cu") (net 10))
 (segment (start 124.03 83.91) (end 124 83.94) (width 0.2) (layer "B.Cu") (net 10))
 (segment (start 131 83.91) (end 131 83.82) (width 0.2) (layer "B.Cu") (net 10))
 (segment (start 131 83.91) (end 124.03 83.91) (width 0.2) (layer "B.Cu") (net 10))
 (segment (start 135.945 84) (end 131.09 84) (width 0.2) (layer "B.Cu") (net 10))
 (segment (start 144.9 90.6) (end 151.5 84) (width 0.2) (layer "F.Cu") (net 15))
 (segment (start 144.9 117.68) (end 144.7 117.88) (width 0.2) (layer "F.Cu") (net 15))
 (segment (start 144.9 90.6) (end 144.9 117.68) (width 0.2) (layer "F.Cu") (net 15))
 (segment (start 156.8 63.68) (end 151.5 63.68) (width 0.2) (layer "B.Cu") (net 23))
 (segment (start 163.5 62.9) (end 157.58 62.9) (width 0.2) (layer "B.Cu") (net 23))
 (segment (start 156.8 63.68) (end 156.8 63.74) (width 0.2) (layer "B.Cu") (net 23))
 (segment (start 157.58 62.9) (end 156.8 63.68) (width 0.2) (layer "B.Cu") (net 23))
 (segment (start 156.3786 68.76) (end 156.74 68.76) (width 0.2) (layer "B.Cu") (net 21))
 (segment (start 162.72 68.76) (end 163.5 67.98) (width 0.2) (layer "B.Cu") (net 21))
 (segment (start 151.5 68.76) (end 156.3786 68.76) (width 0.2) (layer "B.Cu") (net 21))
 (segment (start 156.3786 68.76) (end 162.72 68.76) (width 0.2) (layer "B.Cu") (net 21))
 (segment (start 156.74 68.76) (end 156.8 68.82) (width 0.2) (layer "B.Cu") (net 21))
 (segment (start 149.78 117.88) (end 149.78 90.8) (width 0.2) (layer "F.Cu") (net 13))
 (segment (start 149.78 90.8) (end 151.5 89.08) (width 0.2) (layer "F.Cu") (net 13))
 (segment (start 135.765 78.74) (end 135.945 78.92) (width 0.2) (layer "B.Cu") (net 8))
 (segment (start 130.88 78.86) (end 131 78.74) (width 0.2) (layer "B.Cu") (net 8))
 (segment (start 124 78.86) (end 130.88 78.86) (width 0.2) (layer "B.Cu") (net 8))
 (segment (start 131 78.74) (end 135.765 78.74) (width 0.2) (layer "B.Cu") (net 8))
 (segment (start 151.56 71.36) (end 151.5 71.3) (width 0.2) (layer "B.Cu") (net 20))
 (segment (start 157.64 70.52) (end 156.8 71.36) (width 0.2) (layer "B.Cu") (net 20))
 (segment (start 156.8 71.36) (end 151.56 71.36) (width 0.2) (layer "B.Cu") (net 20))
 (segment (start 163.5 70.52) (end 157.64 70.52) (width 0.2) (layer "B.Cu") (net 20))
 (segment (start 110.2 90.4) (end 105.8 90.4) (width 0.5) (layer "F.Cu") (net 2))
 (segment (start 112.86 114.3) (end 105.5 106.94) (width 0.2) (layer "F.Cu") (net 2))
 (segment (start 114.8 61.7) (end 114.8 85.8) (width 0.5) (layer "F.Cu") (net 2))
 (segment (start 121.4 55.1) (end 114.8 61.7) (width 0.5) (layer "F.Cu") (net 2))
 (segment (start 133.55 57.55) (end 131.1 55.1) (width 0.5) (layer "F.Cu") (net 2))
 (segment (start 105.5 106.94) (end 105.5 90.1) (width 0.2) (layer "F.Cu") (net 2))
 (segment (start 134.2752 115.6048) (end 134.2752 112.0248) (width 0.2) (layer "F.Cu") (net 2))
 (segment (start 134.2752 112.0248) (end 134.3 112) (width 0.2) (layer "F.Cu") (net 2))
 (segment (start 113 119.4) (end 113 114.44) (width 0.2) (layer "F.Cu") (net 2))
 (segment (start 131.1 55.1) (end 121.4 55.1) (width 0.5) (layer "F.Cu") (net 2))
 (segment (start 105.8 90.4) (end 105.5 90.1) (width 0.2) (layer "F.Cu") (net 2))
 (segment (start 132 117.88) (end 134.2752 115.6048) (width 0.2) (layer "F.Cu") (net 2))
 (segment (start 133.55 58.6) (end 133.55 57.55) (width 0.5) (layer "F.Cu") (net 2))
 (segment (start 113 114.44) (end 112.86 114.3) (width 0.2) (layer "F.Cu") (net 2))
 (segment (start 133.55 58.6) (end 135.945 58.6) (width 0.5) (layer "F.Cu") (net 2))
 (segment (start 109.3325 93.9325) (end 105.5 90.1) (width 0.2) (layer "F.Cu") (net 2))
 (segment (start 114.8 85.8) (end 110.2 90.4) (width 0.5) (layer "F.Cu") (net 2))
 (segment (start 109.3325 93.9325) (end 109.3325 96.75) (width 0.2) (layer "F.Cu") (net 2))
 (segment (start 130.48 119.4) (end 113 119.4) (width 0.2) (layer "B.Cu") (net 2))
 (segment (start 132 117.88) (end 130.48 119.4) (width 0.2) (layer "B.Cu") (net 2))
 (segment (start 121.84 107.30865) (end 121.84 117.88) (width 0.2) (layer "F.Cu") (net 27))
 (segment (start 109.3325 99.25) (end 109.3325 99.2) (width 0.2) (layer "F.Cu") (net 27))
 (segment (start 113.73135 99.2) (end 121.84 107.30865) (width 0.2) (layer "F.Cu") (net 27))
 (segment (start 109.3325 99.2) (end 113.73135 99.2) (width 0.2) (layer "F.Cu") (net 27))
 (segment (start 109.3325 102.9017) (end 110.3489 102.9017) (width 0.2) (layer "B.Cu") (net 26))
 (segment (start 124.38 116.9328) (end 124.38 117.88) (width 0.2) (layer "B.Cu") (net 26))
 (segment (start 110.3489 102.9017) (end 124.38 116.9328) (width 0.2) (layer "B.Cu") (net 26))
 (segment (start 109.3325 101.75) (end 109.3325 102.9017) (width 0.2) (layer "B.Cu") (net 26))
 (segment (start 157.64 73.06) (end 156.8 73.9) (width 0.2) (layer "B.Cu") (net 19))
 (segment (start 156.8 73.9) (end 151.56 73.9) (width 0.2) (layer "B.Cu") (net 19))
 (segment (start 163.5 73.06) (end 157.64 73.06) (width 0.2) (layer "B.Cu") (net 19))
 (segment (start 151.56 73.9) (end 151.5 73.84) (width 0.2) (layer "B.Cu") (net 19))
 (segment (start 123.11 122.4063) (end 120.4198 119.7161) (width 0.2) (layer "F.Cu") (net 28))
 (segment (start 126.92 125.5) (end 125.6436 126.7764) (width 0.2) (layer "F.Cu") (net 28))
 (segment (start 123.11 126.0232) (end 123.11 122.4063) (width 0.2) (layer "F.Cu") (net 28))
 (segment (start 125.6436 126.7764) (end 123.8632 126.7764) (width 0.2) (layer "F.Cu") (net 28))
 (segment (start 123.8632 126.7764) (end 123.11 126.0232) (width 0.2) (layer "F.Cu") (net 28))
 (segment (start 120.4198 119.7161) (end 120.4198 116.7798) (width 0.2) (layer "F.Cu") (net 28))
 (segment (start 120.4198 116.7798) (end 117.94 114.3) (width 0.2) (layer "F.Cu") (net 28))
 (segment (start 113.2366 124.2434) (end 128.2034 124.2434) (width 0.2) (layer "B.Cu") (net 25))
 (segment (start 129.46 125.5) (end 132 125.5) (width 0.2) (layer "B.Cu") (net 25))
 (segment (start 113 124.48) (end 113.2366 124.2434) (width 0.2) (layer "B.Cu") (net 25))
 (segment (start 128.2034 124.2434) (end 129.46 125.5) (width 0.2) (layer "B.Cu") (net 25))
 (segment (start 151.5 81.46) (end 156.74 81.46) (width 0.2) (layer "B.Cu") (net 16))
 (segment (start 157.64 80.68) (end 156.8 81.52) (width 0.2) (layer "B.Cu") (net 16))
 (segment (start 163.5 80.68) (end 157.64 80.68) (width 0.2) (layer "B.Cu") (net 16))
 (segment (start 156.74 81.46) (end 156.8 81.52) (width 0.2) (layer "B.Cu") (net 16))
 (segment (start 151.5 78.92) (end 156.3786 78.92) (width 0.2) (layer "B.Cu") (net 17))
 (segment (start 156.3786 78.92) (end 162.72 78.92) (width 0.2) (layer "B.Cu") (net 17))
 (segment (start 156.74 78.92) (end 156.8 78.98) (width 0.2) (layer "B.Cu") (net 17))
 (segment (start 162.72 78.92) (end 163.5 78.14) (width 0.2) (layer "B.Cu") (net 17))
 (segment (start 156.3786 78.92) (end 156.74 78.92) (width 0.2) (layer "B.Cu") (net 17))
 (segment (start 151.5 76.38) (end 156.74 76.38) (width 0.2) (layer "B.Cu") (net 18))
 (segment (start 157.64 75.6) (end 156.8 76.44) (width 0.2) (layer "B.Cu") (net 18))
 (segment (start 163.5 75.6) (end 157.64 75.6) (width 0.2) (layer "B.Cu") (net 18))
 (segment (start 156.74 76.38) (end 156.8 76.44) (width 0.2) (layer "B.Cu") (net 18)))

